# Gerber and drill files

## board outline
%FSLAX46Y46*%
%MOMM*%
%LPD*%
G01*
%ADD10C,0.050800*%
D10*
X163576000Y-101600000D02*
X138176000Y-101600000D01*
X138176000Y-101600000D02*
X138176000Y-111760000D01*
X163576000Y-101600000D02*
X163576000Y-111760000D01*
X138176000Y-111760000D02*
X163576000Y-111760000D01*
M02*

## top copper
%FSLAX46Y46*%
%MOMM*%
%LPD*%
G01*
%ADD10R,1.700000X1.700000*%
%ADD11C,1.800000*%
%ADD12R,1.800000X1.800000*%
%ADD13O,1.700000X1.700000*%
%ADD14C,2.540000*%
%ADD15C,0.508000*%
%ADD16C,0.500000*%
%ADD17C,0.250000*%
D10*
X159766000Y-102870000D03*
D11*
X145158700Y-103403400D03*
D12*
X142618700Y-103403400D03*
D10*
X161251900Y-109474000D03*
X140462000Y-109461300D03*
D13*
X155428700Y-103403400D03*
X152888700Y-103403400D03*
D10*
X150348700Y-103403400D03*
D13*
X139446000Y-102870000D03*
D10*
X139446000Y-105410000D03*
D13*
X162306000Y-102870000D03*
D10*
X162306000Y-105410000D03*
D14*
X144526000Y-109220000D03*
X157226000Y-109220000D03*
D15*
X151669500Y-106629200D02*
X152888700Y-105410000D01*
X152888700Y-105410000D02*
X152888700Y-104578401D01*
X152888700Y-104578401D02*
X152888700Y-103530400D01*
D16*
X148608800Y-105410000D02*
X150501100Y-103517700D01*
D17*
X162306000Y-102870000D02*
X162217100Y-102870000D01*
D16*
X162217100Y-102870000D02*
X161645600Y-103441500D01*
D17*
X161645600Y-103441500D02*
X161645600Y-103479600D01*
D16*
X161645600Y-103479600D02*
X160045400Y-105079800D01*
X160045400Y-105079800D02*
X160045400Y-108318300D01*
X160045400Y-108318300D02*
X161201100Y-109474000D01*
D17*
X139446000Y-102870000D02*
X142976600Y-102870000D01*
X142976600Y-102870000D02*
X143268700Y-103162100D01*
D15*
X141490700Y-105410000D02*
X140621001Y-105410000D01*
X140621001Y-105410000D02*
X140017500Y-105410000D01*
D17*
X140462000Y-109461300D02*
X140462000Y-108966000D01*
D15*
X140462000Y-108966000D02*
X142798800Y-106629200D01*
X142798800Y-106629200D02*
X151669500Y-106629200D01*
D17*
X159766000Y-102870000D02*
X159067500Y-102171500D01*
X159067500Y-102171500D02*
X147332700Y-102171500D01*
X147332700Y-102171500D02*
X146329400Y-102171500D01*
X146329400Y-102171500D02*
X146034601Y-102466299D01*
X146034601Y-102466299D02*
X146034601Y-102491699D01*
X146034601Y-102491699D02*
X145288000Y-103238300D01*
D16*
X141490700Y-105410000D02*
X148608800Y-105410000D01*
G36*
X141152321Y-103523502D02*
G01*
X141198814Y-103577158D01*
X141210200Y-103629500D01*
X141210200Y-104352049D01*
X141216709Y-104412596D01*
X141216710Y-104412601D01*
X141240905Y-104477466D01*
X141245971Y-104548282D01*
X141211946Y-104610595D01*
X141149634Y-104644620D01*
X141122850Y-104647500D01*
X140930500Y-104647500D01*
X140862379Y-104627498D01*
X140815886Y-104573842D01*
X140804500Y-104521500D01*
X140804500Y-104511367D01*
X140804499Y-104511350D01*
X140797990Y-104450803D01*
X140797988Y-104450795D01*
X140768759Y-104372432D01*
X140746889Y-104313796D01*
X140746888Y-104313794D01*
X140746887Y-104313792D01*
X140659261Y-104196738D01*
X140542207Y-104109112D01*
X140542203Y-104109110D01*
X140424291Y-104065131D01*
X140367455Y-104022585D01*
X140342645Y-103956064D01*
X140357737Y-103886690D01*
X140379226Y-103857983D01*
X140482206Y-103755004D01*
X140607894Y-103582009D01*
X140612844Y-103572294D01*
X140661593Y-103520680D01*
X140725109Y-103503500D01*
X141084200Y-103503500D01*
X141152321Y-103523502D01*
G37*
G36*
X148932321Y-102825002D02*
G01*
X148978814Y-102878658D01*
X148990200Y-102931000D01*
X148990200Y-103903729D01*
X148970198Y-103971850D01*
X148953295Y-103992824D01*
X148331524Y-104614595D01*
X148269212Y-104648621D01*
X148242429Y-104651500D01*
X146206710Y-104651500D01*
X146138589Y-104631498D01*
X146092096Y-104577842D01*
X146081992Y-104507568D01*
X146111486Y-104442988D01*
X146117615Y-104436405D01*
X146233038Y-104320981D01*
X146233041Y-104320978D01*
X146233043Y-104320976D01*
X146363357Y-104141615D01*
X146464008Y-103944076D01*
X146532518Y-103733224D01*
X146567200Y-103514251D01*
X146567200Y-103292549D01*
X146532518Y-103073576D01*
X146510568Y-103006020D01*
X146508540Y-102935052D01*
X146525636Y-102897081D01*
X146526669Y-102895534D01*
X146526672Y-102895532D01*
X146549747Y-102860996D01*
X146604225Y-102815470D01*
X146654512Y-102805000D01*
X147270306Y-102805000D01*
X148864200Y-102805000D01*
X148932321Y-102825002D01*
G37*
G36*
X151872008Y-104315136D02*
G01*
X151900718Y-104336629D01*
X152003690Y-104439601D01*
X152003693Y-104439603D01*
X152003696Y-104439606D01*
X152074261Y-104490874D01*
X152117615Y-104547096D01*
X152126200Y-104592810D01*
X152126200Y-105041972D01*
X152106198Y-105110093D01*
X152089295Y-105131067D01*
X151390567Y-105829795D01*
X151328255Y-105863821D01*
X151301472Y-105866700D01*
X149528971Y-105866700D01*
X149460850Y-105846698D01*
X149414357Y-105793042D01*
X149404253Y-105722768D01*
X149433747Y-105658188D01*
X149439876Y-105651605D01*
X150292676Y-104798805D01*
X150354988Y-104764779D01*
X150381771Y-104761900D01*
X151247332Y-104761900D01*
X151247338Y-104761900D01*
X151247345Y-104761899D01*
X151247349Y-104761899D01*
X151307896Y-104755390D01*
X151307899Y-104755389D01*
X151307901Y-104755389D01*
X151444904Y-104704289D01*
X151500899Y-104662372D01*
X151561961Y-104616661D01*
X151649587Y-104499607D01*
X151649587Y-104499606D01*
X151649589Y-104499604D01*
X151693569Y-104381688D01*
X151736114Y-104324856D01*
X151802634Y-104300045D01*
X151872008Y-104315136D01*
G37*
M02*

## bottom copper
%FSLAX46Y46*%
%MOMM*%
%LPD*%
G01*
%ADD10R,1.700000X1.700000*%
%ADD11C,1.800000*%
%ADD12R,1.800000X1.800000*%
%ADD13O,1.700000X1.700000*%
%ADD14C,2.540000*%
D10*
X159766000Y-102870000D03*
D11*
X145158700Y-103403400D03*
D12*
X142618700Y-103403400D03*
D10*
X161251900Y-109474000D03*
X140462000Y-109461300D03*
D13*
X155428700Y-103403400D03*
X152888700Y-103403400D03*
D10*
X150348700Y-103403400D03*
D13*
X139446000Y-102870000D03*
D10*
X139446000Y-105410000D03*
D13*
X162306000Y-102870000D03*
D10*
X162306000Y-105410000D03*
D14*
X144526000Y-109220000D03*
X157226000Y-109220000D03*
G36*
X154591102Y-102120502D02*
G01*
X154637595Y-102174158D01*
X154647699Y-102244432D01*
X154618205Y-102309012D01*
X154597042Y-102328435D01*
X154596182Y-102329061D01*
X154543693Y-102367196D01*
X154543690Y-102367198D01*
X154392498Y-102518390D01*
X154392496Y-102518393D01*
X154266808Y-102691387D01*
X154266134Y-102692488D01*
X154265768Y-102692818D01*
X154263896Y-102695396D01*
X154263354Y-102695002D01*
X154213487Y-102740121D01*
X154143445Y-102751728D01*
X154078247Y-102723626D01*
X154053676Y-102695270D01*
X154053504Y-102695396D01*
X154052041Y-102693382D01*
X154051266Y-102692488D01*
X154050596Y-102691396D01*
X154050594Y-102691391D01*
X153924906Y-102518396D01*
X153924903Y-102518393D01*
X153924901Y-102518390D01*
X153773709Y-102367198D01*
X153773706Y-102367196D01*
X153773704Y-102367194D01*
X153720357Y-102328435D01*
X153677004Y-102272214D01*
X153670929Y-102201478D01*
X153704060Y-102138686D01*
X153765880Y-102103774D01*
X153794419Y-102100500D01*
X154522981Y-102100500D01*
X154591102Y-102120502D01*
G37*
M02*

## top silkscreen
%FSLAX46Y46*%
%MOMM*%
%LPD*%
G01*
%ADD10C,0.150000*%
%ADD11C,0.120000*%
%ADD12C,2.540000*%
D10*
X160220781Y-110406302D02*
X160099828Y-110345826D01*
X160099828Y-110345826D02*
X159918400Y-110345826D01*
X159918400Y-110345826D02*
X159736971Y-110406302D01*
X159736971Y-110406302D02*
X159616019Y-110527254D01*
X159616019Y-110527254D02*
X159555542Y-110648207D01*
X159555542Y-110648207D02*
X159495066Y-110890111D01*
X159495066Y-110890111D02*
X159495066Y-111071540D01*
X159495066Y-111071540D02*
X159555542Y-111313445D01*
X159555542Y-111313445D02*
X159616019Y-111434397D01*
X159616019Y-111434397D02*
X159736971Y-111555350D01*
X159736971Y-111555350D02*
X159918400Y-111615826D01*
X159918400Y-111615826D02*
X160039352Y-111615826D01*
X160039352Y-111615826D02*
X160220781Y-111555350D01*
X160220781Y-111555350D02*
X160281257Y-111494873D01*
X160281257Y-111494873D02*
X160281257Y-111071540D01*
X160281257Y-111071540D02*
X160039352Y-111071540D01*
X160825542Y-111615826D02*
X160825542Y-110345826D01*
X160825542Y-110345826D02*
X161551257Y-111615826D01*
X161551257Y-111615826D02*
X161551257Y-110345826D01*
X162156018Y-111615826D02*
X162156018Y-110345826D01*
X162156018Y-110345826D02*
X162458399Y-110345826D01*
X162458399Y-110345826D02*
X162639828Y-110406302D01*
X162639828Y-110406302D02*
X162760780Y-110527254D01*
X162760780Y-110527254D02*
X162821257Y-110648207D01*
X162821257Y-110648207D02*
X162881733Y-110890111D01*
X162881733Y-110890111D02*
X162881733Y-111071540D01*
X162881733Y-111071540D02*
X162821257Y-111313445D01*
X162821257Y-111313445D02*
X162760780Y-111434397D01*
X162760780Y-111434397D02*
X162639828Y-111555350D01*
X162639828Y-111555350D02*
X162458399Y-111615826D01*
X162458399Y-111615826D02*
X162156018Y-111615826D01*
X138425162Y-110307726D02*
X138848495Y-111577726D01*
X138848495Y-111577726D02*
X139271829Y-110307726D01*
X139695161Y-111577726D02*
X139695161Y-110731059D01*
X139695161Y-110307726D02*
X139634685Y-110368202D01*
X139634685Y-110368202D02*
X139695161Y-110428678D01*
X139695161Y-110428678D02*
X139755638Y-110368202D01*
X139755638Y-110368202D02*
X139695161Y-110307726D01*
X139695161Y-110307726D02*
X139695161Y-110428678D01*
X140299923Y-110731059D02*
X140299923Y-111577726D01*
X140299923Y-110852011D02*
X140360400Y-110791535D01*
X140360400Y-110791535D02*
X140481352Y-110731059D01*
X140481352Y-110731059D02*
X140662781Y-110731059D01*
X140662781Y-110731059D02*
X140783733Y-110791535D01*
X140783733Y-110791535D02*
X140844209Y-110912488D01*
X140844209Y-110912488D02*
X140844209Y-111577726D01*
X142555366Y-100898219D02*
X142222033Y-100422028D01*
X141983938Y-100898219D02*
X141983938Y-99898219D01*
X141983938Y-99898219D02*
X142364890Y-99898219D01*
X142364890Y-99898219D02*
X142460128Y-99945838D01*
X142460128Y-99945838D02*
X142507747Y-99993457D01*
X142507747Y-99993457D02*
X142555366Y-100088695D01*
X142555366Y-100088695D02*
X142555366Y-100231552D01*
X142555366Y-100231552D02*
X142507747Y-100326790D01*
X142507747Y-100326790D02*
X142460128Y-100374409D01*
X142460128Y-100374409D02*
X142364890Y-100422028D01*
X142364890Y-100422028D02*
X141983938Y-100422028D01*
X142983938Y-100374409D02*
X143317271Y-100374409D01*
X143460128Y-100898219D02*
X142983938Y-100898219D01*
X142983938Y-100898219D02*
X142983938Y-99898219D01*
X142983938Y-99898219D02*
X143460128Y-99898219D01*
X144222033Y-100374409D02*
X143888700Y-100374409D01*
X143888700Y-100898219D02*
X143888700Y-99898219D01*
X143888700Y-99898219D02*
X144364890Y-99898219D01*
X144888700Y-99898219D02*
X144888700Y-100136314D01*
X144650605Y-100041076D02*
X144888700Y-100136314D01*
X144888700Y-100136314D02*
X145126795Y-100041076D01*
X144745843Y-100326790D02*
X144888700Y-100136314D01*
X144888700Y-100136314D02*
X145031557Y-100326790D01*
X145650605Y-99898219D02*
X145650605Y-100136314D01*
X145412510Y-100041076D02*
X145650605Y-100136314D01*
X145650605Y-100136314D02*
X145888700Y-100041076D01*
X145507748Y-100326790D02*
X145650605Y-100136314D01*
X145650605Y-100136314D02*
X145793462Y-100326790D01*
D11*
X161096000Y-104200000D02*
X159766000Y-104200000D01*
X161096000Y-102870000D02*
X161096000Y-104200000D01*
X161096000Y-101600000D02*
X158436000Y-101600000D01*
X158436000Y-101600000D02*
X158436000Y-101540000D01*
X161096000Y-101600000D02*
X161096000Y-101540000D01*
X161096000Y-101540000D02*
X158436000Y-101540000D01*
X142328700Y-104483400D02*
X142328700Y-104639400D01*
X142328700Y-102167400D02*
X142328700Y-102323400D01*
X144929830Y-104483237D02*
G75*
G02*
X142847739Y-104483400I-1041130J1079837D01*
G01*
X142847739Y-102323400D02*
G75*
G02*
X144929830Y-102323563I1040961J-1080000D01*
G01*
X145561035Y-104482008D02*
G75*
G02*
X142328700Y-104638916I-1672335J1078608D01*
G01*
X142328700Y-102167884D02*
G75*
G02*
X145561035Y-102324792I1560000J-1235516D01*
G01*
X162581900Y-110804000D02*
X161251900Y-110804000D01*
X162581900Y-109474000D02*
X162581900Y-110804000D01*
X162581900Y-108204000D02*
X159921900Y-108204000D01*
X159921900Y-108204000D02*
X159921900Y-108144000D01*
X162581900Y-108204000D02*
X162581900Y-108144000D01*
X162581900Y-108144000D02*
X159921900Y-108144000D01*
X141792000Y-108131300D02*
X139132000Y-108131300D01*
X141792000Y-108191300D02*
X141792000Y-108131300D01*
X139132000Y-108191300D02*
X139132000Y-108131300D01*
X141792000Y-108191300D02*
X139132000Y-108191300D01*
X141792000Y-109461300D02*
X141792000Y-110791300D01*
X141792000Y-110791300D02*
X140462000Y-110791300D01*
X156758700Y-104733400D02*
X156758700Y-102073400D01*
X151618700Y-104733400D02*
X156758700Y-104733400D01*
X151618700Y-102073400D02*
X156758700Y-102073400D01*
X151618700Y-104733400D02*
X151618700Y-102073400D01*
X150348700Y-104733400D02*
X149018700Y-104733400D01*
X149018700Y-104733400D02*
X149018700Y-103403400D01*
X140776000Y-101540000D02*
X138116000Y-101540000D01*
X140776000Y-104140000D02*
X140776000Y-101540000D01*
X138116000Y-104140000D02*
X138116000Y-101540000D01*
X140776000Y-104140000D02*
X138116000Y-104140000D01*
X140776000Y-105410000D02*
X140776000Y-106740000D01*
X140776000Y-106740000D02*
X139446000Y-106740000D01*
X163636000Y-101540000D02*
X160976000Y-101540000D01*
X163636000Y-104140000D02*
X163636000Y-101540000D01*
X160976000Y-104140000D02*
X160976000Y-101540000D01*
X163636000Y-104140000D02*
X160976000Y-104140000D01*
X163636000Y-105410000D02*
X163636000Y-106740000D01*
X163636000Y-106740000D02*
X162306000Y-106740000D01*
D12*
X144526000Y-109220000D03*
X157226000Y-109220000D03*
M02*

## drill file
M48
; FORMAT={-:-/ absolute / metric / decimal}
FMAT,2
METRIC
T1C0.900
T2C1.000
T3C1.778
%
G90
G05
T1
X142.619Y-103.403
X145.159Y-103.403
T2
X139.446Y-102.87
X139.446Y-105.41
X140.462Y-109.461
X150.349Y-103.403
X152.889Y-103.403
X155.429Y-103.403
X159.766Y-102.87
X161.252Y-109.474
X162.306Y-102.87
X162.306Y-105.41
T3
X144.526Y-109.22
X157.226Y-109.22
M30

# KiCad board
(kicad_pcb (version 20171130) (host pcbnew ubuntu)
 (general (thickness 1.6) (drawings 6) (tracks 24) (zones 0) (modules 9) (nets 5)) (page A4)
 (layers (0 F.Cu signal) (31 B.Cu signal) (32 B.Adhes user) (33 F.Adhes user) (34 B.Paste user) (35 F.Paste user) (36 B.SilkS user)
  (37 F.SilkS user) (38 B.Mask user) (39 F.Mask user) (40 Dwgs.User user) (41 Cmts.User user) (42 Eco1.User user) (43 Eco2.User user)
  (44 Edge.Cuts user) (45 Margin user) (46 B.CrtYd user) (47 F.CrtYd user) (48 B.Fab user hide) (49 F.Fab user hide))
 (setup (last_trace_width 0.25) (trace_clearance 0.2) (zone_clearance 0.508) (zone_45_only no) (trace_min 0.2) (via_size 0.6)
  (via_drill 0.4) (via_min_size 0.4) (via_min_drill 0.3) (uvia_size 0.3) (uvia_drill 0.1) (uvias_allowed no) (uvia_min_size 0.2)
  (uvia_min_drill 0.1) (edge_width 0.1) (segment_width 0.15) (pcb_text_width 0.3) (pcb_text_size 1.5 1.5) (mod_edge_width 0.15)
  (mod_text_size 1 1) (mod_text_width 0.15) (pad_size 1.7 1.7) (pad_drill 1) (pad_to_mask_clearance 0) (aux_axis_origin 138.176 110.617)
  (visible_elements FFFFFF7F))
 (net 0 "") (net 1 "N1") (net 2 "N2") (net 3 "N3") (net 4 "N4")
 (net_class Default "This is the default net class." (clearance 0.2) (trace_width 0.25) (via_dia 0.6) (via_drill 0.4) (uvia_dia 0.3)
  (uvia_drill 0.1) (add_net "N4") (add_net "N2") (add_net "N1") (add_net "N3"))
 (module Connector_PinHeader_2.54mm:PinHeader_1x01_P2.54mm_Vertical (layer F.Cu) (at 159.766 102.87 180)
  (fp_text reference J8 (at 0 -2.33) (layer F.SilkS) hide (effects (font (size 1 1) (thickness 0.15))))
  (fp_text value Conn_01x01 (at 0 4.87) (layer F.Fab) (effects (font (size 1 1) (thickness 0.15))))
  (fp_line (start -1.33 -1.33) (end 0 -1.33) (layer F.SilkS) (width 0.12))
  (fp_line (start -1.33 0) (end -1.33 -1.33) (layer F.SilkS) (width 0.12))
  (fp_line (start -1.33 1.27) (end 1.33 1.27) (layer F.SilkS) (width 0.12))
  (fp_line (start 1.33 1.27) (end 1.33 1.33) (layer F.SilkS) (width 0.12))
  (fp_line (start -1.33 1.27) (end -1.33 1.33) (layer F.SilkS) (width 0.12))
  (fp_line (start -1.33 1.33) (end 1.33 1.33) (layer F.SilkS) (width 0.12))
  (pad 1 thru_hole rect (at 0 0 180) (size 1.7 1.7) (drill 1) (layers *.Cu *.Mask) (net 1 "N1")))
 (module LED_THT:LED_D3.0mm (layer F.Cu) (at 142.6187 103.4034)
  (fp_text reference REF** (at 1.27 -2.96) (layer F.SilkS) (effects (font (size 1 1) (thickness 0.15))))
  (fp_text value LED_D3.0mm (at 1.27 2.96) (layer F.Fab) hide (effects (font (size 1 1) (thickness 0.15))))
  (fp_line (start -0.29 1.08) (end -0.29 1.236) (layer F.SilkS) (width 0.12))
  (fp_line (start -0.29 -1.236) (end -0.29 -1.08) (layer F.SilkS) (width 0.12))
  (fp_arc (start 1.27 0) (end 0.229039 1.08) (angle -87.9) (layer F.SilkS) (width 0.12))
  (fp_arc (start 1.27 0) (end 0.229039 -1.08) (angle 87.9) (layer F.SilkS) (width 0.12))
  (fp_arc (start 1.27 0) (end -0.29 1.235516) (angle -108.8) (layer F.SilkS) (width 0.12))
  (fp_arc (start 1.27 0) (end -0.29 -1.235516) (angle 108.8) (layer F.SilkS) (width 0.12))
  (pad 2 thru_hole circle (at 2.54 0) (size 1.8 1.8) (drill 0.9) (layers *.Cu *.Mask))
  (pad 1 thru_hole rect (at 0 0) (size 1.8 1.8) (drill 0.9) (layers *.Cu *.Mask)))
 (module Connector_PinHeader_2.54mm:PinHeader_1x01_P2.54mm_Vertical (layer F.Cu) (at 161.2519 109.474 180)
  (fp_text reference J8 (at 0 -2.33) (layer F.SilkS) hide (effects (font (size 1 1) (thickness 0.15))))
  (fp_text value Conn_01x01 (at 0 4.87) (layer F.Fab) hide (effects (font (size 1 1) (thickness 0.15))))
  (fp_line (start -1.33 -1.33) (end 0 -1.33) (layer F.SilkS) (width 0.12))
  (fp_line (start -1.33 0) (end -1.33 -1.33) (layer F.SilkS) (width 0.12))
  (fp_line (start -1.33 1.27) (end 1.33 1.27) (layer F.SilkS) (width 0.12))
  (fp_line (start 1.33 1.27) (end 1.33 1.33) (layer F.SilkS) (width 0.12))
  (fp_line (start -1.33 1.27) (end -1.33 1.33) (layer F.SilkS) (width 0.12))
  (fp_line (start -1.33 1.33) (end 1.33 1.33) (layer F.SilkS) (width 0.12))
  (pad 1 thru_hole rect (at 0 0 180) (size 1.7 1.7) (drill 1) (layers *.Cu *.Mask) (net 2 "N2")))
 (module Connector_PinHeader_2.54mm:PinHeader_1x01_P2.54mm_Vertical (layer F.Cu) (at 140.462 109.4613 180)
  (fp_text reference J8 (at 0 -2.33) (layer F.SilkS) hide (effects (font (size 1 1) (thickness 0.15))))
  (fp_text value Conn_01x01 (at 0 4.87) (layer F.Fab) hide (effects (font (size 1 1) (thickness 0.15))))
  (fp_line (start -1.33 1.33) (end 1.33 1.33) (layer F.SilkS) (width 0.12))
  (fp_line (start -1.33 1.27) (end -1.33 1.33) (layer F.SilkS) (width 0.12))
  (fp_line (start 1.33 1.27) (end 1.33 1.33) (layer F.SilkS) (width 0.12))
  (fp_line (start -1.33 1.27) (end 1.33 1.27) (layer F.SilkS) (width 0.12))
  (fp_line (start -1.33 0) (end -1.33 -1.33) (layer F.SilkS) (width 0.12))
  (fp_line (start -1.33 -1.33) (end 0 -1.33) (layer F.SilkS) (width 0.12))
  (pad 1 thru_hole rect (at 0 0 180) (size 1.7 1.7) (drill 1) (layers *.Cu *.Mask) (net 1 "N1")))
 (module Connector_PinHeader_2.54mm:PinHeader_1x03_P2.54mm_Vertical (layer F.Cu) (at 150.3487 103.4034 90)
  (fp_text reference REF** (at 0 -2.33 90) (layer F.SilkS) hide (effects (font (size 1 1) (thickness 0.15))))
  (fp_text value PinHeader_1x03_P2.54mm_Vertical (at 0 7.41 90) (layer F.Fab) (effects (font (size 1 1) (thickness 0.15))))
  (fp_line (start -1.33 6.41) (end 1.33 6.41) (layer F.SilkS) (width 0.12))
  (fp_line (start -1.33 1.27) (end -1.33 6.41) (layer F.SilkS) (width 0.12))
  (fp_line (start 1.33 1.27) (end 1.33 6.41) (layer F.SilkS) (width 0.12))
  (fp_line (start -1.33 1.27) (end 1.33 1.27) (layer F.SilkS) (width 0.12))
  (fp_line (start -1.33 0) (end -1.33 -1.33) (layer F.SilkS) (width 0.12))
  (fp_line (start -1.33 -1.33) (end 0 -1.33) (layer F.SilkS) (width 0.12))
  (pad 3 thru_hole oval (at 0 5.08 90) (size 1.7 1.7) (drill 1) (layers *.Cu *.Mask))
  (pad 2 thru_hole oval (at 0 2.54 90) (size 1.7 1.7) (drill 1) (layers *.Cu *.Mask))
  (pad 1 thru_hole rect (at 0 0 90) (size 1.7 1.7) (drill 1) (layers *.Cu *.Mask)))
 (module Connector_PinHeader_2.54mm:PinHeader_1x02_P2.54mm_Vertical (layer F.Cu) (at 139.446 105.41 180)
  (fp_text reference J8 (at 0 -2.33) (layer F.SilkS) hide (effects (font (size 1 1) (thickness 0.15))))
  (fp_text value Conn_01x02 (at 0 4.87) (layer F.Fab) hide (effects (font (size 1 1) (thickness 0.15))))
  (fp_line (start -1.33 3.87) (end 1.33 3.87) (layer F.SilkS) (width 0.12))
  (fp_line (start -1.33 1.27) (end -1.33 3.87) (layer F.SilkS) (width 0.12))
  (fp_line (start 1.33 1.27) (end 1.33 3.87) (layer F.SilkS) (width 0.12))
  (fp_line (start -1.33 1.27) (end 1.33 1.27) (layer F.SilkS) (width 0.12))
  (fp_line (start -1.33 0) (end -1.33 -1.33) (layer F.SilkS) (width 0.12))
  (fp_line (start -1.33 -1.33) (end 0 -1.33) (layer F.SilkS) (width 0.12))
  (pad 2 thru_hole oval (at 0 2.54 180) (size 1.7 1.7) (drill 1) (layers *.Cu *.Mask) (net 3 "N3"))
  (pad 1 thru_hole rect (at 0 0 180) (size 1.7 1.7) (drill 1) (layers *.Cu *.Mask) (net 1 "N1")))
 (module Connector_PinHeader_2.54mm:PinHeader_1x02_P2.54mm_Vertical (layer F.Cu) (at 162.306 105.41 180)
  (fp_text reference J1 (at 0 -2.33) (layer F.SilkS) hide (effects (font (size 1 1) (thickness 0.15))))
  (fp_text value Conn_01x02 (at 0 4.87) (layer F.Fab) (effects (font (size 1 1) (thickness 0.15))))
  (fp_line (start -1.33 3.87) (end 1.33 3.87) (layer F.SilkS) (width 0.12))
  (fp_line (start -1.33 1.27) (end -1.33 3.87) (layer F.SilkS) (width 0.12))
  (fp_line (start 1.33 1.27) (end 1.33 3.87) (layer F.SilkS) (width 0.12))
  (fp_line (start -1.33 1.27) (end 1.33 1.27) (layer F.SilkS) (width 0.12))
  (fp_line (start -1.33 0) (end -1.33 -1.33) (layer F.SilkS) (width 0.12))
  (fp_line (start -1.33 -1.33) (end 0 -1.33) (layer F.SilkS) (width 0.12))
  (pad 2 thru_hole oval (at 0 2.54 180) (size 1.7 1.7) (drill 1) (layers *.Cu *.Mask) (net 2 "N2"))
  (pad 1 thru_hole rect (at 0 0 180) (size 1.7 1.7) (drill 1) (layers *.Cu *.Mask) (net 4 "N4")))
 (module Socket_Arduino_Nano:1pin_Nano (layer F.Cu) (at 144.526 109.22)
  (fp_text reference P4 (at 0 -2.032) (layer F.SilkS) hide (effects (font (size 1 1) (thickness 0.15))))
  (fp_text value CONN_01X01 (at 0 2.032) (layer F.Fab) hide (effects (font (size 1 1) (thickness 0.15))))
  (pad 1 thru_hole circle (at 0 0) (size 2.54 2.54) (drill 1.778) (layers *.Cu *.Mask F.SilkS)))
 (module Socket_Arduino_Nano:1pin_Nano (layer F.Cu) (at 157.226 109.22)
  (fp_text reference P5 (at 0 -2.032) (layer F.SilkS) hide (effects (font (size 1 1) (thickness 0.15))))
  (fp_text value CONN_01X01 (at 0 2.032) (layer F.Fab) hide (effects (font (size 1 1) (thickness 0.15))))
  (pad 1 thru_hole circle (at 0 0) (size 2.54 2.54) (drill 1.778) (layers *.Cu *.Mask F.SilkS)))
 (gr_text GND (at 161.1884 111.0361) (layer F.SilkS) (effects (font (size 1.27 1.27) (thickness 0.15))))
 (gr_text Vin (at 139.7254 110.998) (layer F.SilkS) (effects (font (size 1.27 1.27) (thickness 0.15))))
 (gr_line (start 163.576 101.6) (end 138.176 101.6) (angle 90) (layer Edge.Cuts) (width 0.0508))
 (gr_line (start 138.176 101.6) (end 138.176 111.76) (angle 90) (layer Edge.Cuts) (width 0.0508))
 (gr_line (start 163.576 101.6) (end 163.576 111.76) (angle 90) (layer Edge.Cuts) (width 0.0508))
 (gr_line (start 138.176 111.76) (end 163.576 111.76) (angle 90) (layer Edge.Cuts) (width 0.0508))
 (segment (start 151.6695 106.6292) (end 152.8887 105.41) (width 0.508) (layer F.Cu) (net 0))
 (segment (start 152.8887 105.41) (end 152.8887 104.578401) (width 0.508) (layer F.Cu) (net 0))
 (segment (start 152.8887 104.578401) (end 152.8887 103.5304) (width 0.508) (layer F.Cu) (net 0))
 (segment (start 148.6088 105.41) (end 150.5011 103.5177) (width 0.5) (layer F.Cu) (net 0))
 (segment (start 162.306 102.87) (end 162.2171 102.87) (width 0.25) (layer F.Cu) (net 2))
 (segment (start 162.2171 102.87) (end 161.6456 103.4415) (width 0.5) (layer F.Cu) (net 2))
 (segment (start 161.6456 103.4415) (end 161.6456 103.4796) (width 0.25) (layer F.Cu) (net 2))
 (segment (start 161.6456 103.4796) (end 160.0454 105.0798) (width 0.5) (layer F.Cu) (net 2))
 (segment (start 160.0454 105.0798) (end 160.0454 108.3183) (width 0.5) (layer F.Cu) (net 2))
 (segment (start 160.0454 108.3183) (end 161.2011 109.474) (width 0.5) (layer F.Cu) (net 2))
 (segment (start 139.446 102.87) (end 142.9766 102.87) (width 0.25) (layer F.Cu) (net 3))
 (segment (start 142.9766 102.87) (end 143.2687 103.1621) (width 0.25) (layer F.Cu) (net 3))
 (segment (start 141.4907 105.41) (end 140.621001 105.41) (width 0.508) (layer F.Cu) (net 1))
 (segment (start 140.621001 105.41) (end 140.0175 105.41) (width 0.508) (layer F.Cu) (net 1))
 (segment (start 140.462 109.4613) (end 140.462 108.966) (width 0.25) (layer F.Cu) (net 1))
 (segment (start 140.462 108.966) (end 142.7988 106.6292) (width 0.508) (layer F.Cu) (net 1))
 (segment (start 142.7988 106.6292) (end 151.6695 106.6292) (width 0.508) (layer F.Cu) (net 1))
 (segment (start 159.766 102.87) (end 159.0675 102.1715) (width 0.25) (layer F.Cu) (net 1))
 (segment (start 159.0675 102.1715) (end 147.3327 102.1715) (width 0.25) (layer F.Cu) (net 1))
 (segment (start 147.3327 102.1715) (end 146.3294 102.1715) (width 0.25) (layer F.Cu) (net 1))
 (segment (start 146.3294 102.1715) (end 146.034601 102.466299) (width 0.25) (layer F.Cu) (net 1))
 (segment (start 146.034601 102.466299) (end 146.034601 102.491699) (width 0.25) (layer F.Cu) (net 1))
 (segment (start 146.034601 102.491699) (end 145.288 103.2383) (width 0.25) (layer F.Cu) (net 1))
 (segment (start 141.4907 105.41) (end 148.6088 105.41) (width 0.5) (layer F.Cu) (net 1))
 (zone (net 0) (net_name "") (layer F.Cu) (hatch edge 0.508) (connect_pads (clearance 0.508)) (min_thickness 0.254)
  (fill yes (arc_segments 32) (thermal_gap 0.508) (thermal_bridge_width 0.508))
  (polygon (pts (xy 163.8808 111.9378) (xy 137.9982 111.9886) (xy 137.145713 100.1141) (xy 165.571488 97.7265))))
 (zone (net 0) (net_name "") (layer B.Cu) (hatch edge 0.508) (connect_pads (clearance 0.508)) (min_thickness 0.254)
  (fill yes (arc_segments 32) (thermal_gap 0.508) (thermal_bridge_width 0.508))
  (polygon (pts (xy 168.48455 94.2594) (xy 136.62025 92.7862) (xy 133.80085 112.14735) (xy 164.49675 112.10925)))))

